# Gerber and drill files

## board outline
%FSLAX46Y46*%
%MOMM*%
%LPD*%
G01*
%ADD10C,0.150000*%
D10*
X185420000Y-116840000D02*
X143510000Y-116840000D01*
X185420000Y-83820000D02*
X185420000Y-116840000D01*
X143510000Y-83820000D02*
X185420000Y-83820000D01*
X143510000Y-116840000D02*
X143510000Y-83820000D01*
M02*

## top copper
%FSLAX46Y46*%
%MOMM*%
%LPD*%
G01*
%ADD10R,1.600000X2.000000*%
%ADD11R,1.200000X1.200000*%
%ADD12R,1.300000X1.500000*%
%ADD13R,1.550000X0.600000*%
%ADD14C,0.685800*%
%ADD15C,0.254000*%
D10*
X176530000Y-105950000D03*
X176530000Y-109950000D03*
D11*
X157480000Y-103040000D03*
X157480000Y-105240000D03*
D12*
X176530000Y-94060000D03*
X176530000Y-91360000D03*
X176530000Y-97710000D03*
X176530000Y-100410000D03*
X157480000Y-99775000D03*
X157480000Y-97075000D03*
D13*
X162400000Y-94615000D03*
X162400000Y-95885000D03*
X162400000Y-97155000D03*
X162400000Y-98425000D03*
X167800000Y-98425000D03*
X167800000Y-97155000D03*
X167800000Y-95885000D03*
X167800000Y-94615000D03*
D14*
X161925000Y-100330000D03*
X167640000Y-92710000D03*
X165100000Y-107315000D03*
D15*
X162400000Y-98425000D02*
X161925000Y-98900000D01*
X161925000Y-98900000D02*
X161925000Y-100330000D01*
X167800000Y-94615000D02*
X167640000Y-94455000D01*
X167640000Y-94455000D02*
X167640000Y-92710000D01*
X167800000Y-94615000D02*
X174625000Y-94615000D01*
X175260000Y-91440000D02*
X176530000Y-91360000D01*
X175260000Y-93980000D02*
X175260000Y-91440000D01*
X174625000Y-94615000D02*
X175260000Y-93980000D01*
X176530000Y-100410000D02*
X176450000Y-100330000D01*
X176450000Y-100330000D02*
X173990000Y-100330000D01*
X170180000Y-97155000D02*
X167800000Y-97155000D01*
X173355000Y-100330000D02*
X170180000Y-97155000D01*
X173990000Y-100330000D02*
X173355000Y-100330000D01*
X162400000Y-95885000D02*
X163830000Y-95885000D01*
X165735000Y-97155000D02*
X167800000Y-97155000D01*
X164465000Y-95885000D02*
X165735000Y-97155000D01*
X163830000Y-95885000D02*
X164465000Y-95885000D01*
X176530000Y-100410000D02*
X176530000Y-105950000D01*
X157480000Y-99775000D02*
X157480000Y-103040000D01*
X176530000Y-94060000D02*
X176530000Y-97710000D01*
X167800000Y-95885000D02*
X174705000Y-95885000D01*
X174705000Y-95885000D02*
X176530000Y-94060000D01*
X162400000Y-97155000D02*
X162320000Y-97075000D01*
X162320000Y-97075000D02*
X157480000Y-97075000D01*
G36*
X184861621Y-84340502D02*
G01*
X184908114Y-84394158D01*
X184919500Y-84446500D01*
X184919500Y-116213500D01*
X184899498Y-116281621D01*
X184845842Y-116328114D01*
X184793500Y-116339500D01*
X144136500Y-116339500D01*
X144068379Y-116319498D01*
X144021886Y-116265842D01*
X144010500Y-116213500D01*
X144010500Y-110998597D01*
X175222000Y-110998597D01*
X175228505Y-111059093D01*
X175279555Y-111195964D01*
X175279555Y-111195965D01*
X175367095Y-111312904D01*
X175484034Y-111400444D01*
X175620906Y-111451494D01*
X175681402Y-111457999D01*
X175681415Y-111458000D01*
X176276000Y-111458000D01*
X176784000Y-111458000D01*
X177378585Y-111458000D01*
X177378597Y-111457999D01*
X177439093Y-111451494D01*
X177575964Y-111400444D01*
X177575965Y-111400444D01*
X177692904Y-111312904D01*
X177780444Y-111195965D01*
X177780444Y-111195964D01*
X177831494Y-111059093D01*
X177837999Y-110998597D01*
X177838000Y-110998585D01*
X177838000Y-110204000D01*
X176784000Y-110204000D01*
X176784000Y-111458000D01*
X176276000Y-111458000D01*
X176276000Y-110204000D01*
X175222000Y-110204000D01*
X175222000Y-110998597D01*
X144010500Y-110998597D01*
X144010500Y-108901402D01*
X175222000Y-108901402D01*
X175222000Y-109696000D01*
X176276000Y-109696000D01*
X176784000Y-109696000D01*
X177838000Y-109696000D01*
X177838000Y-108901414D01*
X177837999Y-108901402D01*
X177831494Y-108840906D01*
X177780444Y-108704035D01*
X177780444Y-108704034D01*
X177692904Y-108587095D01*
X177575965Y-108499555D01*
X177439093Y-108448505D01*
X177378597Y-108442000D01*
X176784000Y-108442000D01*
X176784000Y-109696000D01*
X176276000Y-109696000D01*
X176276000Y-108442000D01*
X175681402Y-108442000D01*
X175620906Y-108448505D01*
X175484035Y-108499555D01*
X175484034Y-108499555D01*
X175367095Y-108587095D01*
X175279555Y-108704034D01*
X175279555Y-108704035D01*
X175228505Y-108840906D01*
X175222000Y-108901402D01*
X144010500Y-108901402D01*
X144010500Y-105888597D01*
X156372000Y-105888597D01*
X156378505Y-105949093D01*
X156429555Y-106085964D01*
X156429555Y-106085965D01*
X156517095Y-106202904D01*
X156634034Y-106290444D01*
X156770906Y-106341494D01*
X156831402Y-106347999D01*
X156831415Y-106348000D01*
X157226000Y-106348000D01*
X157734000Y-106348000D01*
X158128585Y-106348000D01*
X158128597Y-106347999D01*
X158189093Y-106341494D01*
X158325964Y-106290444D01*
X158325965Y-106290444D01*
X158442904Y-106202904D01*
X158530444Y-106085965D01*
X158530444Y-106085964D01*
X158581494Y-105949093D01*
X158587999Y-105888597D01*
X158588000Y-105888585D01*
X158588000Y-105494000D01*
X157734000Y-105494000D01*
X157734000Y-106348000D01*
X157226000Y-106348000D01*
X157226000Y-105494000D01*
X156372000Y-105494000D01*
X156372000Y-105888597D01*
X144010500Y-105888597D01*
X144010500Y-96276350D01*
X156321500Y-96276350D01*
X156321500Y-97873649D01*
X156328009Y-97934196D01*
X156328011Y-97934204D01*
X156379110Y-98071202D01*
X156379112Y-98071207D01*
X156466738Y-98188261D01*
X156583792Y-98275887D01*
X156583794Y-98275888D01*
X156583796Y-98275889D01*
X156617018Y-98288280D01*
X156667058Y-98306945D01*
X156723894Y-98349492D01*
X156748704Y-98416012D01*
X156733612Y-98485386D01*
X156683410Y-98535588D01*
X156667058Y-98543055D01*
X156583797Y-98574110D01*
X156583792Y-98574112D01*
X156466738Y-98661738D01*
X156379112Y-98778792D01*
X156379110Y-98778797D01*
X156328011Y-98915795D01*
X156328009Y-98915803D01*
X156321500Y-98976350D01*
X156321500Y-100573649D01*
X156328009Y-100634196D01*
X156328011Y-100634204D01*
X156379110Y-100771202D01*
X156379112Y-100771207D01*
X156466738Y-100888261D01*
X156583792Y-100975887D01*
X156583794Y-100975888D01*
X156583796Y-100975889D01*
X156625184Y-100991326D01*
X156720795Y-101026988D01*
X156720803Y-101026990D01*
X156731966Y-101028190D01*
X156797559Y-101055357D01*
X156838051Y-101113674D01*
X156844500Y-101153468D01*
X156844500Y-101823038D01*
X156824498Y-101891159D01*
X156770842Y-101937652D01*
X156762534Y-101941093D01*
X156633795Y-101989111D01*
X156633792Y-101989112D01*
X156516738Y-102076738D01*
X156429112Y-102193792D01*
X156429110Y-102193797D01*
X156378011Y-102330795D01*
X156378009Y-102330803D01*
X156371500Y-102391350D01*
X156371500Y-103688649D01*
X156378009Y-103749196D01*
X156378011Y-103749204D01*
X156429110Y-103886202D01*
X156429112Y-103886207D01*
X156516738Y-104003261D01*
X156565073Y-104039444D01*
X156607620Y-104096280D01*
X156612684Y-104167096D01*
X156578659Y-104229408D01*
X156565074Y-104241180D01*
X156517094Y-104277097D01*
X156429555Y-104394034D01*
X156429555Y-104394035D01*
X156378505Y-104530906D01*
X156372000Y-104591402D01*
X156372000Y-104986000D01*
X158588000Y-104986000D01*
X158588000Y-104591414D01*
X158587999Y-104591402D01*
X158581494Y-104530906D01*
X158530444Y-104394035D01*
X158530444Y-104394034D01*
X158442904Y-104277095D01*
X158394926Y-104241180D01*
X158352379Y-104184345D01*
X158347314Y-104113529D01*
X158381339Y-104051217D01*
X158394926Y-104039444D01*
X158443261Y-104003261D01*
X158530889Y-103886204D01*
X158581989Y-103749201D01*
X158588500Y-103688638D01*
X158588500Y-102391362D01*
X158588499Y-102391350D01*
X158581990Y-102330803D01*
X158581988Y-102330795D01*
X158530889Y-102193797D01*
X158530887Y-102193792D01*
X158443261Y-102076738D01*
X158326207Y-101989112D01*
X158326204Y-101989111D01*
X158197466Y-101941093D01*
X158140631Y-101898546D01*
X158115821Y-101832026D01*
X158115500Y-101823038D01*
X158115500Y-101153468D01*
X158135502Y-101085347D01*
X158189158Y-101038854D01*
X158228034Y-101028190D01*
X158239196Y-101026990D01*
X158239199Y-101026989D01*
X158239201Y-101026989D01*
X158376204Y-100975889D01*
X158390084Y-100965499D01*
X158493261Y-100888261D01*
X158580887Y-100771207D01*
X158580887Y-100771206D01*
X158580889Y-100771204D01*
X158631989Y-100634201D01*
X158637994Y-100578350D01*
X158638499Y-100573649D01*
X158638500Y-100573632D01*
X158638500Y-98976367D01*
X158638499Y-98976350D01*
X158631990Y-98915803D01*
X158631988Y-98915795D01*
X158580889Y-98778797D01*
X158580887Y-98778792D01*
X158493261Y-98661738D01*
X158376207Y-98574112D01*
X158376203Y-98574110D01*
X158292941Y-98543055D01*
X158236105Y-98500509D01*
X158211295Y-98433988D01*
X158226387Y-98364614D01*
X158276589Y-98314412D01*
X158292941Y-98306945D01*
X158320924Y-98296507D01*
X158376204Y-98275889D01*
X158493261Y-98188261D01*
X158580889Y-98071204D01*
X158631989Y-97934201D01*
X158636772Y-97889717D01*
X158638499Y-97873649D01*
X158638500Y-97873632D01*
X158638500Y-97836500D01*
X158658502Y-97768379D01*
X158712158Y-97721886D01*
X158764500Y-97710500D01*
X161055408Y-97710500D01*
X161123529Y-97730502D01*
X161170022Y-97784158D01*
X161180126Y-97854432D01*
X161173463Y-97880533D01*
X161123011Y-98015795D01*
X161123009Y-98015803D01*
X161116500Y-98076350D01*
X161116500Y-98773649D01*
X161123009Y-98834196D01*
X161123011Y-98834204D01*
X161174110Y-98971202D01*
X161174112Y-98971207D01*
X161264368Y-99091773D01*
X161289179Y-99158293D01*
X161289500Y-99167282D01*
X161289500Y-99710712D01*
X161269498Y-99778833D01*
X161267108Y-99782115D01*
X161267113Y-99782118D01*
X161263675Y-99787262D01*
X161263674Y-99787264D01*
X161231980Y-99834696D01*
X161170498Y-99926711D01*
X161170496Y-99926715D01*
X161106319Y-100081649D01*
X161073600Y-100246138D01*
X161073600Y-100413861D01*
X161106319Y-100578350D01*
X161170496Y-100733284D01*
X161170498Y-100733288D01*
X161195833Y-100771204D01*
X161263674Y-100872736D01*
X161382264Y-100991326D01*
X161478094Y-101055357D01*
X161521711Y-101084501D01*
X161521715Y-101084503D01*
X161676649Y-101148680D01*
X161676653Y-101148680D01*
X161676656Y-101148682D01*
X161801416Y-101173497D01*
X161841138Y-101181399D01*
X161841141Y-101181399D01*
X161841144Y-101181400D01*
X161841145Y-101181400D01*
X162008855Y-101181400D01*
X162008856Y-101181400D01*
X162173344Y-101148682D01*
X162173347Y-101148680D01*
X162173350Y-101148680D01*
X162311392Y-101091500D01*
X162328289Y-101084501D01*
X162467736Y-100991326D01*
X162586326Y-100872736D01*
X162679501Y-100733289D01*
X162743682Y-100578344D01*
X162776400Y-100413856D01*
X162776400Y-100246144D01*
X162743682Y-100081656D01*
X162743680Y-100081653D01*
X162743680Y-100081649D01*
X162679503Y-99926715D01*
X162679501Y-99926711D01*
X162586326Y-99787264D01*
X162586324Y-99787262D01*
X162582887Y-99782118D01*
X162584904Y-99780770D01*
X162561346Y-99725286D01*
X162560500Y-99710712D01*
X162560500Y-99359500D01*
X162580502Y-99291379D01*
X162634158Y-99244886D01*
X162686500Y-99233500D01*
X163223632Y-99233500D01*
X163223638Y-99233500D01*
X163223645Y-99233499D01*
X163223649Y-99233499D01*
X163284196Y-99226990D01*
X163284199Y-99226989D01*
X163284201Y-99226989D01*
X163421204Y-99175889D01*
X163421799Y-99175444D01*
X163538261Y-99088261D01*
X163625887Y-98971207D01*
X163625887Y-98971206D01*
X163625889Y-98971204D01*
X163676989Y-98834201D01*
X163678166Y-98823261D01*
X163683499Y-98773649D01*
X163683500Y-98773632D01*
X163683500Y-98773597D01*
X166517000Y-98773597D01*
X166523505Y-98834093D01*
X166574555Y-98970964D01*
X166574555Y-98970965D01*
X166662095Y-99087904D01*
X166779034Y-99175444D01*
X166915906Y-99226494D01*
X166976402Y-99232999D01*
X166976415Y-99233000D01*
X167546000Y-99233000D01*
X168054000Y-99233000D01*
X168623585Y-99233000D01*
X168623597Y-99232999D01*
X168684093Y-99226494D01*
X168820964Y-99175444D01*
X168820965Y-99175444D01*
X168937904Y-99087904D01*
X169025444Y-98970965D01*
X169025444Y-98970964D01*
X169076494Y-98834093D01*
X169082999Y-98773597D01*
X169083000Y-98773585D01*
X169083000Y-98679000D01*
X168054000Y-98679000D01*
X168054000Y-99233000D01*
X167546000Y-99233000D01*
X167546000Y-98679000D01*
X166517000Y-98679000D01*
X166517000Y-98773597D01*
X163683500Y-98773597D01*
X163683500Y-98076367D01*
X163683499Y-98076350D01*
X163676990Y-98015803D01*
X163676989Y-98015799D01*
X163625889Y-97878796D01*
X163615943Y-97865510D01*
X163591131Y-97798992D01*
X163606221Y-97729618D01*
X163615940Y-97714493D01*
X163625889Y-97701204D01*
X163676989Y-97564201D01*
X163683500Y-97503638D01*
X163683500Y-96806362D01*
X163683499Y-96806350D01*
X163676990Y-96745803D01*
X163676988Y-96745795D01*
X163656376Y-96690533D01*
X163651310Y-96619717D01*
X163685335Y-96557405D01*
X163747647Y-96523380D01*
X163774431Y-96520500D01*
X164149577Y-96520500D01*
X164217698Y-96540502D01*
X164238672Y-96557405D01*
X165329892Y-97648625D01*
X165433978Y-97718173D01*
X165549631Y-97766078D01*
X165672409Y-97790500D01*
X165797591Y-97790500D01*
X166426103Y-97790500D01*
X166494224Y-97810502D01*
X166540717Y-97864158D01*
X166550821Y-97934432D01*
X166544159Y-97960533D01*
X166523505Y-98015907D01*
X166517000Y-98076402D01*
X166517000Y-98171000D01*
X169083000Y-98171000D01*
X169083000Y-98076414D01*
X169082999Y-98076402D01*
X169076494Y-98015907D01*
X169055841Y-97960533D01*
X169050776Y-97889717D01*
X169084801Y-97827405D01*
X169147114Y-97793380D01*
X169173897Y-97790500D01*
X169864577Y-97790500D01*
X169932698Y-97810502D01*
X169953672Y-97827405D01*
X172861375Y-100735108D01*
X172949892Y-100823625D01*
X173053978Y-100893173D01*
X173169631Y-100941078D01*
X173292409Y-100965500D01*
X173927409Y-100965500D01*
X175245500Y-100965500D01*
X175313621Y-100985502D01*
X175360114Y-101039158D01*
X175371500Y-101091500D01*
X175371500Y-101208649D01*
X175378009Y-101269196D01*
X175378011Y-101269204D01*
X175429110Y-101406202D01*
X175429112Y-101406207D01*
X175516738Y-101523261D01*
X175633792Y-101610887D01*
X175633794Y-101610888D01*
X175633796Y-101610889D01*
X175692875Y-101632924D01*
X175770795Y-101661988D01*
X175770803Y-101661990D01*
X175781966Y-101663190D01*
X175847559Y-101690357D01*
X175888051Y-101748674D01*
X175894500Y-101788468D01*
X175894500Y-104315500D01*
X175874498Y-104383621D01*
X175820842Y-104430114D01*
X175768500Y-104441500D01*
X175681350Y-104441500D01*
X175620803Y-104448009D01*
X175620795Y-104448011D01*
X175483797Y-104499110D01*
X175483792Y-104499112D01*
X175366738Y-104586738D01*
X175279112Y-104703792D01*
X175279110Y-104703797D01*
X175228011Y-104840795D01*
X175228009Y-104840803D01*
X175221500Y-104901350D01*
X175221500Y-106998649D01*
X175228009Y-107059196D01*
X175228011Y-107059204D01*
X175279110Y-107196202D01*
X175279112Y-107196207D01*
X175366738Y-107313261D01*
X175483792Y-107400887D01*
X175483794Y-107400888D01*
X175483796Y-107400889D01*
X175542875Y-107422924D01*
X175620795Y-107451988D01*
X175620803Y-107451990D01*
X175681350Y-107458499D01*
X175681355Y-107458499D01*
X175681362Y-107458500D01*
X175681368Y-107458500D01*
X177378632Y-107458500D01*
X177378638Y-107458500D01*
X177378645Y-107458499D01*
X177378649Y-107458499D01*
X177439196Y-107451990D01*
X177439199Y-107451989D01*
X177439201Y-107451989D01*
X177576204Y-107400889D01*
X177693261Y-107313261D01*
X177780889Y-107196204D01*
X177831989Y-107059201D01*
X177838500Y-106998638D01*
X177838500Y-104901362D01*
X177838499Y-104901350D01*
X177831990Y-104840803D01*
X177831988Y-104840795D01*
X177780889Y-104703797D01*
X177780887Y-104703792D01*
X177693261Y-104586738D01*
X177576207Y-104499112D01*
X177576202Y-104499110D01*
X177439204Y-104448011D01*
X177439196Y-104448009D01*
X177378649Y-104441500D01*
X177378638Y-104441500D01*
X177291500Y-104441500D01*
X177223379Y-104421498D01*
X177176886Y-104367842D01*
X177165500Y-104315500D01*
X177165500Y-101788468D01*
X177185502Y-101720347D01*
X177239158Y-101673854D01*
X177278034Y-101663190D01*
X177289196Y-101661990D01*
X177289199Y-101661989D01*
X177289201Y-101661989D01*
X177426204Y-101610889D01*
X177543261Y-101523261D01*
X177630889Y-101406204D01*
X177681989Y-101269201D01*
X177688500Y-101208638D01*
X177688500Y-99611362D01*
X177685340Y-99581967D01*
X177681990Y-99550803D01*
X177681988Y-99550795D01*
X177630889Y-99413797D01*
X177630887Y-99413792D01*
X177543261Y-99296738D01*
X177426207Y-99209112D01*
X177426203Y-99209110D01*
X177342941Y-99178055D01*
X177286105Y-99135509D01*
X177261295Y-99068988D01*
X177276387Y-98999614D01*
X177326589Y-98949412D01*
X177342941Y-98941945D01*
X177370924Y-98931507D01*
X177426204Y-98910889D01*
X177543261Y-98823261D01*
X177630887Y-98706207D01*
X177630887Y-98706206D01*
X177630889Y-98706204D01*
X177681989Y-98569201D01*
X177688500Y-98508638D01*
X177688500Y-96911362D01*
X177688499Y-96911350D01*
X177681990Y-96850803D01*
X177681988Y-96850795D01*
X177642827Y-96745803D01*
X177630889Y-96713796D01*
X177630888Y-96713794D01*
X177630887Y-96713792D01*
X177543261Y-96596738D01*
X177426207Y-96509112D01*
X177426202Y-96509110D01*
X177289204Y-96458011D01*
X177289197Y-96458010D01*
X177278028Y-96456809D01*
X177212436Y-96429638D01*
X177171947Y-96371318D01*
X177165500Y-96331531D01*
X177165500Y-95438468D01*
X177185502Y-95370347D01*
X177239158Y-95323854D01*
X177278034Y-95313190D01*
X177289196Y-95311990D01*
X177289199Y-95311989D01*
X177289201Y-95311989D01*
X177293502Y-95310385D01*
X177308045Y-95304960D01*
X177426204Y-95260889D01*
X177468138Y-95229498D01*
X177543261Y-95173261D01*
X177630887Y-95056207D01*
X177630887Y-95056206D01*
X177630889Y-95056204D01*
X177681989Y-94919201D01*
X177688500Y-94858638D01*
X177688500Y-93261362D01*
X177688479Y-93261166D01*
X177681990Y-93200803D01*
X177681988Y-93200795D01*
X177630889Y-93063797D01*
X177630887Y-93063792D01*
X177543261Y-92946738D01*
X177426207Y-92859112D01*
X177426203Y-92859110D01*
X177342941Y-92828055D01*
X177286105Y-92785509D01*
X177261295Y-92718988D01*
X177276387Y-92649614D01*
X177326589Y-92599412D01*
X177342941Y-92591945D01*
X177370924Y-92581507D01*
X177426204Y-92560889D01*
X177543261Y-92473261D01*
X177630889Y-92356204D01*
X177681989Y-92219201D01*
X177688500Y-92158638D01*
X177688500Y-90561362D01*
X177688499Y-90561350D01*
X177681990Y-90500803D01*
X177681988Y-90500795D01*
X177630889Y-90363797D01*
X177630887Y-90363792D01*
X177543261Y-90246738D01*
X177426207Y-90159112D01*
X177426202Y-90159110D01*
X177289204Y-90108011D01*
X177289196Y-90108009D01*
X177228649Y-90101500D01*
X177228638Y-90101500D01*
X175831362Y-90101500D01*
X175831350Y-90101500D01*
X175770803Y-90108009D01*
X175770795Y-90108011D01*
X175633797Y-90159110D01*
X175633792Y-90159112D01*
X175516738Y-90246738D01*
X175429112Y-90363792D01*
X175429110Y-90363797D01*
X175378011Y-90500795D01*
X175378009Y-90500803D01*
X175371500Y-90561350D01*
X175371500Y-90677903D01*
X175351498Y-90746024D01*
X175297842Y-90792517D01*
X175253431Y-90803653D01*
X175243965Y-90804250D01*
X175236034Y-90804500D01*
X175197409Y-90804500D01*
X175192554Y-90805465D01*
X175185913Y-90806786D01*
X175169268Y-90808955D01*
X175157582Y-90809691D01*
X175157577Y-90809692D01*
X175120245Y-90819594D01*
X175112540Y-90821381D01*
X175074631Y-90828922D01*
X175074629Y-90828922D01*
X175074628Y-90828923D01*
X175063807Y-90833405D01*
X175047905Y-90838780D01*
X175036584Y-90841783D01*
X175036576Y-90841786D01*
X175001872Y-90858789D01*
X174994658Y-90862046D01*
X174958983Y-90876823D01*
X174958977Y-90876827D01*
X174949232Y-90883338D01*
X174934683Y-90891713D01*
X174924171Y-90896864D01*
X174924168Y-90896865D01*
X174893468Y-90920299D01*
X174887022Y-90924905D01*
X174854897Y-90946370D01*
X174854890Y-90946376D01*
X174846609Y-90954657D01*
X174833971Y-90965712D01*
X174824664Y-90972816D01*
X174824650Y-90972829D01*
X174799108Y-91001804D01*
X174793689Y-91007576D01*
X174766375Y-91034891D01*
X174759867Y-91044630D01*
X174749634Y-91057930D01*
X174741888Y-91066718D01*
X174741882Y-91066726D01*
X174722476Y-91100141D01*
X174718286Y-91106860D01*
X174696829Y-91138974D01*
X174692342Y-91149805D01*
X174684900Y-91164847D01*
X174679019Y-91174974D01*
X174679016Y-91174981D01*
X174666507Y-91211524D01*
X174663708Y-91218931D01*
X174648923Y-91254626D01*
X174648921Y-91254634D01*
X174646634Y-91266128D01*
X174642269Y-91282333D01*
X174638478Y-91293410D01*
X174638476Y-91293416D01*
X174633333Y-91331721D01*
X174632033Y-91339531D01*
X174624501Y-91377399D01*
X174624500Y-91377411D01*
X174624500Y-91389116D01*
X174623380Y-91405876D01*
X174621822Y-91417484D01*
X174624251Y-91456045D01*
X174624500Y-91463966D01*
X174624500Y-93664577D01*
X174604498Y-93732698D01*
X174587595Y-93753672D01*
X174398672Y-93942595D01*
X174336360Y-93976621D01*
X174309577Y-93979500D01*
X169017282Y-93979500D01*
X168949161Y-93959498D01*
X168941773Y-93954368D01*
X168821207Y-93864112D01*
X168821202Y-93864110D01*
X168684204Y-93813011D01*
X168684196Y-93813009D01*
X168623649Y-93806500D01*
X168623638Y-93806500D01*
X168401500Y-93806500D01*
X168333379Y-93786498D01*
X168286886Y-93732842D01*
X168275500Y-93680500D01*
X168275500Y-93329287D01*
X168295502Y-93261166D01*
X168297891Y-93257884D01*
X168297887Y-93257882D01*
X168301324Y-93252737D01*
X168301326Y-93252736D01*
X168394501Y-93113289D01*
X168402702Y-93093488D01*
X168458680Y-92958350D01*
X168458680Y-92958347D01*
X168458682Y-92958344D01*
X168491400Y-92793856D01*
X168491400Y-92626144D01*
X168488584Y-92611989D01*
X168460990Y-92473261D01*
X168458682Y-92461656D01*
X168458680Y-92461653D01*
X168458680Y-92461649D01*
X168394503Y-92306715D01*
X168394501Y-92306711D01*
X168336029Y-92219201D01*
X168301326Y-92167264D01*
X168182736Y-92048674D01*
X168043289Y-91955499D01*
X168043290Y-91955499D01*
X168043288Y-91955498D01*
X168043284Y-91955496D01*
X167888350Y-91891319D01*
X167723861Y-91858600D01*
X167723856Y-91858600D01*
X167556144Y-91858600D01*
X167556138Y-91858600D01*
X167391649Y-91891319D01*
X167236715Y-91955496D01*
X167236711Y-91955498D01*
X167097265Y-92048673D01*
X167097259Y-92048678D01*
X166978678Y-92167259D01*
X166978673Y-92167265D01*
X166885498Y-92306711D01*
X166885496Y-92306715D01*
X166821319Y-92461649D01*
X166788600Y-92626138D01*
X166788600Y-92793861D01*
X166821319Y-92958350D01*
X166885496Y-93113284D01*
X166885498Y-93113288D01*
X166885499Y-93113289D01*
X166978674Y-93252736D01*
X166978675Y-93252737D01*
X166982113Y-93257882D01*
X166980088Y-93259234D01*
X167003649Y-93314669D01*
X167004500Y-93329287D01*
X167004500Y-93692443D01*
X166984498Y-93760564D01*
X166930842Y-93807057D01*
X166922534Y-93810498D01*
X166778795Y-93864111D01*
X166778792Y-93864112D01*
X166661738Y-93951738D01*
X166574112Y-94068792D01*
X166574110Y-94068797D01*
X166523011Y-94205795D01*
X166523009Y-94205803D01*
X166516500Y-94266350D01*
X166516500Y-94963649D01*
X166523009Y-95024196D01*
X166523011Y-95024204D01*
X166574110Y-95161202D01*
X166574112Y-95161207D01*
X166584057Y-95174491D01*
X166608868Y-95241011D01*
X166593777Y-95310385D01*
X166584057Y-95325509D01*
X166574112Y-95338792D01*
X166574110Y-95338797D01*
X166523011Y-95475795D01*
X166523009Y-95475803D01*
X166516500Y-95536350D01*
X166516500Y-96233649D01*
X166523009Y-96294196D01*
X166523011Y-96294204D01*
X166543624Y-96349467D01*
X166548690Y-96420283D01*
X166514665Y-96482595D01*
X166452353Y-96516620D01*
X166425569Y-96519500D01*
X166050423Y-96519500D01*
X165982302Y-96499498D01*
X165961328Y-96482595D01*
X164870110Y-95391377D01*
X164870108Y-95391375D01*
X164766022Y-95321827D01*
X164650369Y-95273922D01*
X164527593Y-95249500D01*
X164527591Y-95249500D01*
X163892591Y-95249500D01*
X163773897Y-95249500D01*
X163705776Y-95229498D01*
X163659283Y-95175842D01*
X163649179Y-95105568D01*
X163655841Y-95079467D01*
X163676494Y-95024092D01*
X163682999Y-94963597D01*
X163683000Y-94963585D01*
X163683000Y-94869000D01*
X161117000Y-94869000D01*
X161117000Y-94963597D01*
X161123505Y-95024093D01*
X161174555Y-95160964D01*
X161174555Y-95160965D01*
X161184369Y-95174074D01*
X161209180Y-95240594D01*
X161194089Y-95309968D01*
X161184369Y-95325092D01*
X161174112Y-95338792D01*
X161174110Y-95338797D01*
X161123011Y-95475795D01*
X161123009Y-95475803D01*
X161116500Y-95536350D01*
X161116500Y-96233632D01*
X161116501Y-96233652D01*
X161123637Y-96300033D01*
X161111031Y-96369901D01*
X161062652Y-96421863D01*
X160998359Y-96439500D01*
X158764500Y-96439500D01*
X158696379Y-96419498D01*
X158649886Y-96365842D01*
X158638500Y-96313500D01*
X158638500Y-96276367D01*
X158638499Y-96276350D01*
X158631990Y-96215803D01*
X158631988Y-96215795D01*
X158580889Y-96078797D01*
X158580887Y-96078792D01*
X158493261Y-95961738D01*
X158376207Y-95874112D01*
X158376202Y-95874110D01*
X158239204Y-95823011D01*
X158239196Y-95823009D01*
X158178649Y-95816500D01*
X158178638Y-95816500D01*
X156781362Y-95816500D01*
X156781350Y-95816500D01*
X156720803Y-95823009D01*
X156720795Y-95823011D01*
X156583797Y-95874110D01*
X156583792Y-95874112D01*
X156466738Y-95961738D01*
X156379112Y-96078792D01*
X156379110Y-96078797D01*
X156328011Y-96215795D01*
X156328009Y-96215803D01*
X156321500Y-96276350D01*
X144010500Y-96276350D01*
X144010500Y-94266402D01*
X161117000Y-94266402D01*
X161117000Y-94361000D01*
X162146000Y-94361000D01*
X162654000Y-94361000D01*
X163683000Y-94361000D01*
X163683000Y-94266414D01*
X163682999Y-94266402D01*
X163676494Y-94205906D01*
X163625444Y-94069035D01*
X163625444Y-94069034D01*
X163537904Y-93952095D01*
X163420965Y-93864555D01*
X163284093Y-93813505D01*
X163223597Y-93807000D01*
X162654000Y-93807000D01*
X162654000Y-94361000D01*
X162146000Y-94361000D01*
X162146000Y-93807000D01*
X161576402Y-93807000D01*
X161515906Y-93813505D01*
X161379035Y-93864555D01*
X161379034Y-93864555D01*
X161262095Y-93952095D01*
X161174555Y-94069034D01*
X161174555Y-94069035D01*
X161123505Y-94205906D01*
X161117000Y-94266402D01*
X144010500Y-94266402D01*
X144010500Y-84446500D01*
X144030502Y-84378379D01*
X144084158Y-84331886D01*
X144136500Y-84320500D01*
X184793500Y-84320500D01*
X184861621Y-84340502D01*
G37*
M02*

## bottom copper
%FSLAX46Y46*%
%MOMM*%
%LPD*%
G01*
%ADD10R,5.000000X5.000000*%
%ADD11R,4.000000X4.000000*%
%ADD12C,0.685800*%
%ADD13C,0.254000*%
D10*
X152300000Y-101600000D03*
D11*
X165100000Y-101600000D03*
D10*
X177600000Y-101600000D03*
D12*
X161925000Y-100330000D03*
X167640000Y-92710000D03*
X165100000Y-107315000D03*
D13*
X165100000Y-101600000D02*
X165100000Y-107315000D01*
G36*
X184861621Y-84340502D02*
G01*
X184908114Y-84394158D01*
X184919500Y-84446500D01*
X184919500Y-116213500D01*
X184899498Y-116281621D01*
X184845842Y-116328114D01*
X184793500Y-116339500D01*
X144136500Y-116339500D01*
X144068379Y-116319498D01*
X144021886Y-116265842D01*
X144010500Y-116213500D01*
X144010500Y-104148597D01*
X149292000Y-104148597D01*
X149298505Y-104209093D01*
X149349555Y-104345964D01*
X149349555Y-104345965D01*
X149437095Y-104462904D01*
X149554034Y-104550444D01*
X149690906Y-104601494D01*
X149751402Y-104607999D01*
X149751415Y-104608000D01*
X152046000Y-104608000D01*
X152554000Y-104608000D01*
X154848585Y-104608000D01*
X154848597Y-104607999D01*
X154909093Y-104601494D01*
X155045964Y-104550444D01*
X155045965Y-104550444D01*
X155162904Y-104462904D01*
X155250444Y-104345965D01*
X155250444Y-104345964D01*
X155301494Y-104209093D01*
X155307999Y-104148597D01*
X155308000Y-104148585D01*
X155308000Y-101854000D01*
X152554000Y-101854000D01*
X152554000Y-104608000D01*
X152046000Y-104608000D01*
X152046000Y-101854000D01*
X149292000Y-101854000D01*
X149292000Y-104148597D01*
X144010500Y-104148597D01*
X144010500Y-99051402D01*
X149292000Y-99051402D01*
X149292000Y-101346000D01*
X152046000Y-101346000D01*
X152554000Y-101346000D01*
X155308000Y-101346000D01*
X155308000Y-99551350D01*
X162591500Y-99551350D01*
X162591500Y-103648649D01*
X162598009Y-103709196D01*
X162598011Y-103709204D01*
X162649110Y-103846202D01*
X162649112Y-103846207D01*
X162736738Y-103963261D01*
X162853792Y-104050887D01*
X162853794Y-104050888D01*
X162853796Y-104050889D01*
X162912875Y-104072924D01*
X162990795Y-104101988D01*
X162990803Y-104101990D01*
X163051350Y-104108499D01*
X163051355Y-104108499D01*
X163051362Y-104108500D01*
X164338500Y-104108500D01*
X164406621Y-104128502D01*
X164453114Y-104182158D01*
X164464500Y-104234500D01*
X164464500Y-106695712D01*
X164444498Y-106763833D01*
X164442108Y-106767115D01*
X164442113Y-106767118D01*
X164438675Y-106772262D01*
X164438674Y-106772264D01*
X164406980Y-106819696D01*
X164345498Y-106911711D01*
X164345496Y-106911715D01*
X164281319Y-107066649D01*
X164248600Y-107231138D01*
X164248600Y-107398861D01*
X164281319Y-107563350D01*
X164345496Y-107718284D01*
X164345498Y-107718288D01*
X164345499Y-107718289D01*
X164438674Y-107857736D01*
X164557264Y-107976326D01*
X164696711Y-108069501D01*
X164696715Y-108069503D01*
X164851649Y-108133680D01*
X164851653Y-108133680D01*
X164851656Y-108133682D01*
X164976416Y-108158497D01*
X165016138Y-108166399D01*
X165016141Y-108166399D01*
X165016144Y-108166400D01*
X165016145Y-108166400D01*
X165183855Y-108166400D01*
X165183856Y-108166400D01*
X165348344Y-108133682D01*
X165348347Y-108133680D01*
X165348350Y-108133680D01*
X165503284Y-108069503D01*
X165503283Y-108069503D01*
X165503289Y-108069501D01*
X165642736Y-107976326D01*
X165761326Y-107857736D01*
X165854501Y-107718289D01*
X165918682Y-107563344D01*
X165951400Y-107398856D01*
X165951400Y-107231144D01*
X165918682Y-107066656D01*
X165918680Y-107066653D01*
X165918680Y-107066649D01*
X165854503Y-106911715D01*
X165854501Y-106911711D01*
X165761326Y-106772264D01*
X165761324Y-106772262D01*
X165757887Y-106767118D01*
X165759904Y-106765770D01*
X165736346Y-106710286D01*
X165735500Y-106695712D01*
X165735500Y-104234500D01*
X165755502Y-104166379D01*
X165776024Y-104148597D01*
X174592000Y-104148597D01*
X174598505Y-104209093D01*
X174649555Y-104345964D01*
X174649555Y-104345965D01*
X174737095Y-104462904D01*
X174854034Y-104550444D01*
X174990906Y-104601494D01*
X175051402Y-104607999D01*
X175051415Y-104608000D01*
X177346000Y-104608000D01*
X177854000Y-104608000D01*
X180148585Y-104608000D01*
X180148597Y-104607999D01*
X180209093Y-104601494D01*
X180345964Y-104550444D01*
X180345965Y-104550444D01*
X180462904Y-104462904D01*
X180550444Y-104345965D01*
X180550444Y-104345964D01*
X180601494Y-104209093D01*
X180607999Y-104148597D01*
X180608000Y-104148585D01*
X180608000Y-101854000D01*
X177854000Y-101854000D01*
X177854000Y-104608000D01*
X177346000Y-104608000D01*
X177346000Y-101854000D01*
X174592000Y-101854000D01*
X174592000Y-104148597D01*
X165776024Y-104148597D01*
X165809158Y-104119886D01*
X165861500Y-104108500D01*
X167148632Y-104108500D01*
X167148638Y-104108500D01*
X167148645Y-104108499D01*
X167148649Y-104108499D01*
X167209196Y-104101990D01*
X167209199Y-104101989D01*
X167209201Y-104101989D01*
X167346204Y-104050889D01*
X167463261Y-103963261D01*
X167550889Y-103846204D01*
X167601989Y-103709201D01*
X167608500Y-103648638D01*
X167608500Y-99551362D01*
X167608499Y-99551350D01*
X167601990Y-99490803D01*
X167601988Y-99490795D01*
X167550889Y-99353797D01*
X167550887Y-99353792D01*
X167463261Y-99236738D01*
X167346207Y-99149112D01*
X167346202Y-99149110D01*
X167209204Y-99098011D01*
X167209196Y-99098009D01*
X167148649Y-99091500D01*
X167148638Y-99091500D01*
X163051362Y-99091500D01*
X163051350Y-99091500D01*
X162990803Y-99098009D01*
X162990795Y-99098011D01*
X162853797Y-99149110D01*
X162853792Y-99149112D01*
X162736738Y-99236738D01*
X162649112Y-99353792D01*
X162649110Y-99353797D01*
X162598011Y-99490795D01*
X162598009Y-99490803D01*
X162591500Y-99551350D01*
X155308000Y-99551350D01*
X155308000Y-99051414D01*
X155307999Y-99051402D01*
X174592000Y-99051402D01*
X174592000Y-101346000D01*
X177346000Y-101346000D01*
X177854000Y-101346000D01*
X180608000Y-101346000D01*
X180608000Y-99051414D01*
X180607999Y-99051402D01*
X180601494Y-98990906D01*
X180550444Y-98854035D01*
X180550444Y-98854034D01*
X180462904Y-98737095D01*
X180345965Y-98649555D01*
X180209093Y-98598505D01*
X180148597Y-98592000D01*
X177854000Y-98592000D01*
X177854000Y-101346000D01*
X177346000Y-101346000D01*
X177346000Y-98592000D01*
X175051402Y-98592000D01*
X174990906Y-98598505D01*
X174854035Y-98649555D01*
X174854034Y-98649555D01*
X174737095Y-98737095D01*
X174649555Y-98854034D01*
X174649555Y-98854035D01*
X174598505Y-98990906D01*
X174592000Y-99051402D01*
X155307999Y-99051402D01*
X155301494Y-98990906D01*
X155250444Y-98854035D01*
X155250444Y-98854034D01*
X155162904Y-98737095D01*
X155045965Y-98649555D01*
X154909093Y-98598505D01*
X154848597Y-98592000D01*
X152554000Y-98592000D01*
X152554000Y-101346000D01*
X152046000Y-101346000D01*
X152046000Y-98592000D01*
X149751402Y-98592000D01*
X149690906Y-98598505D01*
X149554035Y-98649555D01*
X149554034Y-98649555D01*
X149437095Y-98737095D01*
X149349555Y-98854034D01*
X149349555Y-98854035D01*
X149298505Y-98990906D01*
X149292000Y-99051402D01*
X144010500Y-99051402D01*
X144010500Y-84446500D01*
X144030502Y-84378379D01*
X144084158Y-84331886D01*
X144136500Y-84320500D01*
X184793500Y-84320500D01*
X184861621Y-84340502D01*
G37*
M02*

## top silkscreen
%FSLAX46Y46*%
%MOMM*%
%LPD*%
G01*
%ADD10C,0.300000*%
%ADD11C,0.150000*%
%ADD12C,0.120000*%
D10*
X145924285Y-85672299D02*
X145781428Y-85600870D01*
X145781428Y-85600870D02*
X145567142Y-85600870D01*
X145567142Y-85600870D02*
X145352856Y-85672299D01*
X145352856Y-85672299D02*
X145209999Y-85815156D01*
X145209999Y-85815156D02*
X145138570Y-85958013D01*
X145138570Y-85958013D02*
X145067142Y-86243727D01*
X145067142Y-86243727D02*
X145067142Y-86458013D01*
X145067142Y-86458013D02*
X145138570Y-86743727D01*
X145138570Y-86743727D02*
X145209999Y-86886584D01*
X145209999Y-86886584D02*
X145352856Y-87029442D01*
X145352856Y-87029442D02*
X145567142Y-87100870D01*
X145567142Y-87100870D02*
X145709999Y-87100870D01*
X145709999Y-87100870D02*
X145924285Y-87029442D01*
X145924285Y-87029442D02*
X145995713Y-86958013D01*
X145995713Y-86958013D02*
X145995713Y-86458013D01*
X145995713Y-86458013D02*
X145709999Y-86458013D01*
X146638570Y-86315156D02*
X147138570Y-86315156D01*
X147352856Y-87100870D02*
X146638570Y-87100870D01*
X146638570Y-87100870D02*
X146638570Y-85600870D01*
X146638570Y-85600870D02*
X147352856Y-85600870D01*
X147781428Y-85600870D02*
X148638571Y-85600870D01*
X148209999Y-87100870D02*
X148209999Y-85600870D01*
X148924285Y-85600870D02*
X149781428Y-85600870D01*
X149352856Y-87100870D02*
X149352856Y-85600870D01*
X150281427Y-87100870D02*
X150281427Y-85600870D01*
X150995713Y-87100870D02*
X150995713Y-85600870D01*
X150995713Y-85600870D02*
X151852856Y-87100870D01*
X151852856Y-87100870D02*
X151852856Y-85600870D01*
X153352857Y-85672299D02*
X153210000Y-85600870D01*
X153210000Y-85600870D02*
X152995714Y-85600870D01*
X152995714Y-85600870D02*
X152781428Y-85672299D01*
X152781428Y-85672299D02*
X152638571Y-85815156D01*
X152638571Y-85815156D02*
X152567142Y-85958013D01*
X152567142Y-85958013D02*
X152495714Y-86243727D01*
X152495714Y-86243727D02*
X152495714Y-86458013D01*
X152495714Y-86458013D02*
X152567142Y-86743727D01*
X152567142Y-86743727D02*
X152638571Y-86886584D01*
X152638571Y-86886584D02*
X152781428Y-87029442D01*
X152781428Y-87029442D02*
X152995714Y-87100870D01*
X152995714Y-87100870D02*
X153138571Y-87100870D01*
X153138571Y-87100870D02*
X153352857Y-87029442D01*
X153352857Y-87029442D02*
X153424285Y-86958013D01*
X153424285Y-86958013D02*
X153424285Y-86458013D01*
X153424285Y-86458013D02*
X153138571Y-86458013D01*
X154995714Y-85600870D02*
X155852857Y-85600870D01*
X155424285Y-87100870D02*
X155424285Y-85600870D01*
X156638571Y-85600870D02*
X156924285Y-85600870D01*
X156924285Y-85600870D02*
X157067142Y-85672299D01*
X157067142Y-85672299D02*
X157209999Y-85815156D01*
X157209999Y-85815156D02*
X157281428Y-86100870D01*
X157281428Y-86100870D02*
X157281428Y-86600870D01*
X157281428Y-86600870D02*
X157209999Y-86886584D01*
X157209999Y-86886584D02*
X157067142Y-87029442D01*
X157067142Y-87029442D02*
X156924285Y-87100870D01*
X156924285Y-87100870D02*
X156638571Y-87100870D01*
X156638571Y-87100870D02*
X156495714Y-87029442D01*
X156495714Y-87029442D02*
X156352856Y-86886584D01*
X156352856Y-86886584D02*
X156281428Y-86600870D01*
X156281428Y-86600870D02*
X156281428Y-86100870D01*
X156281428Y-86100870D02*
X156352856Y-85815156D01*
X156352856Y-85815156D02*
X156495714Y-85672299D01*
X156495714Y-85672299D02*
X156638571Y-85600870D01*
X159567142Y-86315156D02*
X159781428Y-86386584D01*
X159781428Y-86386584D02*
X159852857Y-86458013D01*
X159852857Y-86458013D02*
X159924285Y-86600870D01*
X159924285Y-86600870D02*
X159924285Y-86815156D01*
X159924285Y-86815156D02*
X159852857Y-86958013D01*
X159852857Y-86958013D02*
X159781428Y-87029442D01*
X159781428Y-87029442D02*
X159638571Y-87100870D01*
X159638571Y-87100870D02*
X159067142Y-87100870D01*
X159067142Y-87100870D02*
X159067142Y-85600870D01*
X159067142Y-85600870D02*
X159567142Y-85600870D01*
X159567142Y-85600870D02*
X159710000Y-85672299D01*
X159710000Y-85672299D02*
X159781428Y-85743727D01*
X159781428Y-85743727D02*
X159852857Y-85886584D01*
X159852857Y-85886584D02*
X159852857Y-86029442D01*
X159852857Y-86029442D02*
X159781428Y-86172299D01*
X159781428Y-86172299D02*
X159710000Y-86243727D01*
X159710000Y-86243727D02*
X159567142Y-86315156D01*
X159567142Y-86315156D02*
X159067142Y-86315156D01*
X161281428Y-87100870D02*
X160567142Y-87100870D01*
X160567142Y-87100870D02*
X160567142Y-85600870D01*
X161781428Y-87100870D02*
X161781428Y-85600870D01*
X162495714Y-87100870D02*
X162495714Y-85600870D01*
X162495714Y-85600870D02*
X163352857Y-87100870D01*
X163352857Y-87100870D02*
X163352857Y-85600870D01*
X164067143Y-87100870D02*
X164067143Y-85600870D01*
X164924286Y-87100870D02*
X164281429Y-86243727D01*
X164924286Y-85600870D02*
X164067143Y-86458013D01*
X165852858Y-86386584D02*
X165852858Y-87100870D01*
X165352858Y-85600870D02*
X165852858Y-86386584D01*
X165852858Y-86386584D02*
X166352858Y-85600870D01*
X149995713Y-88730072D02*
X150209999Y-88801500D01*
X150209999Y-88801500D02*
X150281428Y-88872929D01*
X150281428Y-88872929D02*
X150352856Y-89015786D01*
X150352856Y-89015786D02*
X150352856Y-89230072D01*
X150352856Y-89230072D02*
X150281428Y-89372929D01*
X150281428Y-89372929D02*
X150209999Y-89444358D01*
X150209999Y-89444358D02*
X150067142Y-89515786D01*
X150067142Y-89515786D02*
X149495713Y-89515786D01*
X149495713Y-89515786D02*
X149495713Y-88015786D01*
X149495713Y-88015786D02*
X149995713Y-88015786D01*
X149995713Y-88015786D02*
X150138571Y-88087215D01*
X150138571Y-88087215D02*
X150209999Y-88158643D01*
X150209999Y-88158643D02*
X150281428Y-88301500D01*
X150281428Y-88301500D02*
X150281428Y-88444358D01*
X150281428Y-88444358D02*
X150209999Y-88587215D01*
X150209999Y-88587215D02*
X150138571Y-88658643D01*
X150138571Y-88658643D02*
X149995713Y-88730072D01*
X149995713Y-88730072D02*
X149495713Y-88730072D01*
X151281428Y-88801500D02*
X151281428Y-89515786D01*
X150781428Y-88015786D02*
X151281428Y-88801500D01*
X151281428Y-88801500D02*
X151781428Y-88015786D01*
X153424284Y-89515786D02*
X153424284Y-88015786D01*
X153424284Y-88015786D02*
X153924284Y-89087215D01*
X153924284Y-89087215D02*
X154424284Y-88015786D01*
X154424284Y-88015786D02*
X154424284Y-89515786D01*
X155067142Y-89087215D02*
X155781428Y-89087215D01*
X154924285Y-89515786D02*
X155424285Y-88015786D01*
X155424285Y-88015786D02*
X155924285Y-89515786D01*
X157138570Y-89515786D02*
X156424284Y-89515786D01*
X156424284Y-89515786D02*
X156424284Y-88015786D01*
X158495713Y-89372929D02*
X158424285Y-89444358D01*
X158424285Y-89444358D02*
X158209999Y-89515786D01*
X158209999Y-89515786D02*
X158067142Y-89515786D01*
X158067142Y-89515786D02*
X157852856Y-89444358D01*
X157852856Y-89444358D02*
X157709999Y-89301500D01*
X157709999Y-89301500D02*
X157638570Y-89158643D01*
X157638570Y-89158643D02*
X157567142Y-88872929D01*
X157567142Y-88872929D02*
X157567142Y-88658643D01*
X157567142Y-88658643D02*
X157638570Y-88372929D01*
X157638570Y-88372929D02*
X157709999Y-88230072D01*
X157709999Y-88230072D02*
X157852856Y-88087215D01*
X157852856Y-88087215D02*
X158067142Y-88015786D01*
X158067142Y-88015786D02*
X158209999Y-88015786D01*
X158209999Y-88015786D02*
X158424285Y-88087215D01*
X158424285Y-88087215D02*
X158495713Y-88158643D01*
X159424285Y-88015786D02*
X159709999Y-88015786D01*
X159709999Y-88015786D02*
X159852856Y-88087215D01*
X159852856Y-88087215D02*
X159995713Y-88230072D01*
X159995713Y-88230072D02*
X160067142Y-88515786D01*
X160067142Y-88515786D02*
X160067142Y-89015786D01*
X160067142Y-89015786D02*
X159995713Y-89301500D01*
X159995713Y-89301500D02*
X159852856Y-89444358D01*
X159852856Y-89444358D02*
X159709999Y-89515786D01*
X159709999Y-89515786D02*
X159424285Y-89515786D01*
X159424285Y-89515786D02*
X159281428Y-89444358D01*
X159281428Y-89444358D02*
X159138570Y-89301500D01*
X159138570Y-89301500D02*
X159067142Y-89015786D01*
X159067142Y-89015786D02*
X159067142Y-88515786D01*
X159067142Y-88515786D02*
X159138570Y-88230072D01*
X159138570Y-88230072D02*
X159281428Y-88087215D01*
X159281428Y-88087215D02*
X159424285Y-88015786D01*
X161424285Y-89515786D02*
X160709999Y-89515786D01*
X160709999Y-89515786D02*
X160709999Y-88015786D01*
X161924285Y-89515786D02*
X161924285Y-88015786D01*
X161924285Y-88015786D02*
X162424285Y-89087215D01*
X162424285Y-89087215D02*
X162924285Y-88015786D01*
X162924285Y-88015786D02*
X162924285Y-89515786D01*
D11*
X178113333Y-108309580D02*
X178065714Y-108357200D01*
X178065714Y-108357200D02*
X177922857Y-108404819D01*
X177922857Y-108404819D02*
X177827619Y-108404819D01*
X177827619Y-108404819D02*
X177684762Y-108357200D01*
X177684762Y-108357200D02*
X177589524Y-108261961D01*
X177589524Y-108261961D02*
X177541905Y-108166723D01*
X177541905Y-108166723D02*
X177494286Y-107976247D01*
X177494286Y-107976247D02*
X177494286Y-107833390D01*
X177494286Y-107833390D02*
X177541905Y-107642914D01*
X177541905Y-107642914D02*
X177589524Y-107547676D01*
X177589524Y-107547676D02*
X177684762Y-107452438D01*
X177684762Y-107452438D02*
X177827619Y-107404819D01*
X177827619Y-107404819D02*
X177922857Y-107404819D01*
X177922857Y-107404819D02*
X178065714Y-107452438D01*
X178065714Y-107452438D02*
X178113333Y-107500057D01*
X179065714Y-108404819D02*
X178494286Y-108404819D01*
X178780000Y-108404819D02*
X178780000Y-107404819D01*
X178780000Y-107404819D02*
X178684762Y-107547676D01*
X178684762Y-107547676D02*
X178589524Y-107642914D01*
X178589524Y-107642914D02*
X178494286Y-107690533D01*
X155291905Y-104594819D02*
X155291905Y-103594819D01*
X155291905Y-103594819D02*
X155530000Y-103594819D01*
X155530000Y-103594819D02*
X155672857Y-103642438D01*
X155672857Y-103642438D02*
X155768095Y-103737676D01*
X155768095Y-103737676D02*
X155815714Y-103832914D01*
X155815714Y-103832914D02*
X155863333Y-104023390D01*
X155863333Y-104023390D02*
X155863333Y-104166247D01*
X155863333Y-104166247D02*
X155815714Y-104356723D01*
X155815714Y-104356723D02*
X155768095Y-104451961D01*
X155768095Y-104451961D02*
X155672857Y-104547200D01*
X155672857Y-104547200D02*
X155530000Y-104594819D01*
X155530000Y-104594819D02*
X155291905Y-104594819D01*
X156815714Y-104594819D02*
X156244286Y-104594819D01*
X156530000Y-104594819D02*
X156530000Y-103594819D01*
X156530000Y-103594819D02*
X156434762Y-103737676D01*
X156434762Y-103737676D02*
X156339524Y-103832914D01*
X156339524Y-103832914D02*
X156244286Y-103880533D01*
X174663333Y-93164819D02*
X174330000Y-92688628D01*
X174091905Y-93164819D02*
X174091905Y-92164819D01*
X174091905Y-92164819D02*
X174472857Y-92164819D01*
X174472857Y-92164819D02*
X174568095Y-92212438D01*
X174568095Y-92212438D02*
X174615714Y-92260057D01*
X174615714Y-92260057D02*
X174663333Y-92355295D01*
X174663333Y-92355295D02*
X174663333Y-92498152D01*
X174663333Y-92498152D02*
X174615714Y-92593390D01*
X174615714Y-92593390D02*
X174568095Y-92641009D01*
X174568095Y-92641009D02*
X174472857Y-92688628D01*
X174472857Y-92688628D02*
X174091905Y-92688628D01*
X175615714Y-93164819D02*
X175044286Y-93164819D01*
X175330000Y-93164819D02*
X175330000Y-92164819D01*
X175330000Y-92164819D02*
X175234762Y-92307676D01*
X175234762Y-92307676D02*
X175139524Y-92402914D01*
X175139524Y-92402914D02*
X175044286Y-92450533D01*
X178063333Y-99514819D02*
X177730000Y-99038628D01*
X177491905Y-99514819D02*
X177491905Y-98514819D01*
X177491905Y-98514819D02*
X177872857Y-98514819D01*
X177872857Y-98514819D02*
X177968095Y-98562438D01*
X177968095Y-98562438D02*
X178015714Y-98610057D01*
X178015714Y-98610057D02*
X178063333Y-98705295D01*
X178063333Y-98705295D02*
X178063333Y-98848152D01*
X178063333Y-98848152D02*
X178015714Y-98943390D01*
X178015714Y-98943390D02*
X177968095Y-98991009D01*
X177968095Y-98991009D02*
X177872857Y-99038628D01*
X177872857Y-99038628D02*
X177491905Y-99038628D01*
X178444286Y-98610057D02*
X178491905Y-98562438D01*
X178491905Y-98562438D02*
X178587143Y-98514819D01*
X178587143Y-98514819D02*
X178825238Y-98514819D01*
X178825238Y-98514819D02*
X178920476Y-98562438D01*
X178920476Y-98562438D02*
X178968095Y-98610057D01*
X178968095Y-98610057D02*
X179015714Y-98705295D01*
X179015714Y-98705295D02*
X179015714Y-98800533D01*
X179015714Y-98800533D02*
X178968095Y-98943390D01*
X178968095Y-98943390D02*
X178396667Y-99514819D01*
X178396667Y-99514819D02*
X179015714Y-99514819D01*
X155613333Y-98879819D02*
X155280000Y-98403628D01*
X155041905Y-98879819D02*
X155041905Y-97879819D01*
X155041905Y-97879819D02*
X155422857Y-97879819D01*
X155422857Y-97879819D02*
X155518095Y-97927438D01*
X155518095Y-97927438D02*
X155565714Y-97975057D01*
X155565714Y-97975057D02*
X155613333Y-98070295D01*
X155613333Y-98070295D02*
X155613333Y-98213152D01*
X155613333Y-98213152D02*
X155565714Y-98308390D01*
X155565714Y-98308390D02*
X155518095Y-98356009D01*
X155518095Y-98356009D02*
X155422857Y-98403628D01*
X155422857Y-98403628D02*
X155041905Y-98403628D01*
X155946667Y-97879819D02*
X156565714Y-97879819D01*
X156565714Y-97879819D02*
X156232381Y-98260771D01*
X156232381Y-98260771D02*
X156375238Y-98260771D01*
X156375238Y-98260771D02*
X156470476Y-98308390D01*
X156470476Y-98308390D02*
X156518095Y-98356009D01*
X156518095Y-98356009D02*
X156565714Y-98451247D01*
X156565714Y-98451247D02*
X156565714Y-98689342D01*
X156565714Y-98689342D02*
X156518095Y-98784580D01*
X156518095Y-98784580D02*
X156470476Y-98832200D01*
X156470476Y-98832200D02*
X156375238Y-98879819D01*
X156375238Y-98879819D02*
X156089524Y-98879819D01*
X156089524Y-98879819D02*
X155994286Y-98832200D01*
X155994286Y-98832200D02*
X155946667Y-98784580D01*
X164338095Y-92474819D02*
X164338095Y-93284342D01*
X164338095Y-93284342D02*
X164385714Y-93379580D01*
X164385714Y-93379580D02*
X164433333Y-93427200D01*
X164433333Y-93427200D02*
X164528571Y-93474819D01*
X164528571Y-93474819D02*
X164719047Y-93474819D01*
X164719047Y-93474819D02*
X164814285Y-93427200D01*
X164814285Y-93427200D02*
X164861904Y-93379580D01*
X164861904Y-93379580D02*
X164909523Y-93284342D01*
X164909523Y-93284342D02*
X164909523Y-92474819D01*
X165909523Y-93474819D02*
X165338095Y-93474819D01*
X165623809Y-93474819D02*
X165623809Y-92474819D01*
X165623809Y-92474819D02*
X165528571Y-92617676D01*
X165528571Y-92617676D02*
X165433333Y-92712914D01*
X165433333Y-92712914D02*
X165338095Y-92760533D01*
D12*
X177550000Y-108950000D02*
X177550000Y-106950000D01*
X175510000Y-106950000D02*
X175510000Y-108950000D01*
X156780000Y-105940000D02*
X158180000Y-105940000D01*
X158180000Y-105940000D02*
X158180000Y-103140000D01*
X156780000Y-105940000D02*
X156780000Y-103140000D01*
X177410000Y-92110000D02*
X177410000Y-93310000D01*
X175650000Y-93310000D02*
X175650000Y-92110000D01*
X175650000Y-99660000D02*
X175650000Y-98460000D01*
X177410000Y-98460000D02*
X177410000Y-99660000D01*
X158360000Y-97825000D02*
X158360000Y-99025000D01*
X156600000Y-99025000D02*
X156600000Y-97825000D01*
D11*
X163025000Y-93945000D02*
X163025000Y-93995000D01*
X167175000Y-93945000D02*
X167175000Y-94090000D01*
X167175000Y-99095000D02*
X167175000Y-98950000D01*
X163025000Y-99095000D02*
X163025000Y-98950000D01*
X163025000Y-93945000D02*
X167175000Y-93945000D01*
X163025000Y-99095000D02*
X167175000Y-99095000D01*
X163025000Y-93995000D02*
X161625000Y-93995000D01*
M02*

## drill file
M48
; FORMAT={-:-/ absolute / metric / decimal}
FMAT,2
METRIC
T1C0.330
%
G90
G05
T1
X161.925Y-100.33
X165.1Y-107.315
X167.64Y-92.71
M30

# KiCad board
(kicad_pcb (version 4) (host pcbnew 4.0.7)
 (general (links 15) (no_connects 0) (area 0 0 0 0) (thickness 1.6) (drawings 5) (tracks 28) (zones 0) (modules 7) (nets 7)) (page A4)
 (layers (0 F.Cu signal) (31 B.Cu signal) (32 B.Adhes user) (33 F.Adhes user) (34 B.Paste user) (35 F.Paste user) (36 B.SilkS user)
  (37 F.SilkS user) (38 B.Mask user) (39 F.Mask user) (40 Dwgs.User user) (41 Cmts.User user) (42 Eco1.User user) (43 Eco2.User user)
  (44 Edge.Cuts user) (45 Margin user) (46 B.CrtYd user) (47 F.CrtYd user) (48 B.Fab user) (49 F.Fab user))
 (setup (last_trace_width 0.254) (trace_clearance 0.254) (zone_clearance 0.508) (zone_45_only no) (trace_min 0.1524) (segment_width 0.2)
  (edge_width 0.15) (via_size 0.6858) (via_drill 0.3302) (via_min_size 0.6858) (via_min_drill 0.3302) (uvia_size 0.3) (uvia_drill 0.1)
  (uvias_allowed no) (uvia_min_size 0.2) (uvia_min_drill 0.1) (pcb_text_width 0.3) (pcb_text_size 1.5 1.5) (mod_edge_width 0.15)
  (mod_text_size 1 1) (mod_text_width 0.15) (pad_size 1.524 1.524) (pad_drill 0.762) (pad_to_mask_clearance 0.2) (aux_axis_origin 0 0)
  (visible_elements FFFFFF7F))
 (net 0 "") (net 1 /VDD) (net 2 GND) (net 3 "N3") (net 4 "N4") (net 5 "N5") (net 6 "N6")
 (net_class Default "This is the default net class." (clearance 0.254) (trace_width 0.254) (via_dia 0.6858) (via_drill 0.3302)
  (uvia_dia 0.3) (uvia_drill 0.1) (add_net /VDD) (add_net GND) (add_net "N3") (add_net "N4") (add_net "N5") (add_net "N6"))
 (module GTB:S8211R (layer B.Cu) (at 165.1 101.6)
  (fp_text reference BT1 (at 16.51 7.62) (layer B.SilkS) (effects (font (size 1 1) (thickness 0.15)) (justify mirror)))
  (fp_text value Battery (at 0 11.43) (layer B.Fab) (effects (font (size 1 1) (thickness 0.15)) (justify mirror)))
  (pad 1 smd rect (at -12.8 0) (size 5 5) (layers B.Cu B.Paste B.Mask) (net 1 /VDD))
  (pad 2 smd rect (at 0 0) (size 4 4) (layers B.Cu B.Paste B.Mask) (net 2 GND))
  (pad 1 smd rect (at 12.5 0) (size 5 5) (layers B.Cu B.Paste B.Mask) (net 1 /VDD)))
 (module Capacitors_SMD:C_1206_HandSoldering (layer F.Cu) (at 176.53 107.95 270)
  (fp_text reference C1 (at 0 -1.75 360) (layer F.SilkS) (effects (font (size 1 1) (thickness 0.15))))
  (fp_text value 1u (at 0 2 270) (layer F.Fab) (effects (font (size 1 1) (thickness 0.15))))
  (fp_line (start 1 -1.02) (end -1 -1.02) (layer F.SilkS) (width 0.12))
  (fp_line (start -1 1.02) (end 1 1.02) (layer F.SilkS) (width 0.12))
  (pad 1 smd rect (at -2 0 270) (size 2 1.6) (layers F.Cu F.Paste F.Mask) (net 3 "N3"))
  (pad 2 smd rect (at 2 0 270) (size 2 1.6) (layers F.Cu F.Paste F.Mask) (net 2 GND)))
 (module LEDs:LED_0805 (layer F.Cu) (at 157.48 104.14 90)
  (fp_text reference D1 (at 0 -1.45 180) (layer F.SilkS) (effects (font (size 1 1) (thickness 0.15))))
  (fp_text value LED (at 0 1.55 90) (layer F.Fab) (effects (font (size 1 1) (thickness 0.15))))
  (fp_line (start -1.8 -0.7) (end -1.8 0.7) (layer F.SilkS) (width 0.12))
  (fp_line (start -1.8 0.7) (end 1 0.7) (layer F.SilkS) (width 0.12))
  (fp_line (start -1.8 -0.7) (end 1 -0.7) (layer F.SilkS) (width 0.12))
  (pad 2 smd rect (at 1.1 0 270) (size 1.2 1.2) (layers F.Cu F.Paste F.Mask) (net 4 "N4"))
  (pad 1 smd rect (at -1.1 0 270) (size 1.2 1.2) (layers F.Cu F.Paste F.Mask) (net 2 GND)))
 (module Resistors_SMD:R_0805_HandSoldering (layer F.Cu) (at 176.53 92.71 90)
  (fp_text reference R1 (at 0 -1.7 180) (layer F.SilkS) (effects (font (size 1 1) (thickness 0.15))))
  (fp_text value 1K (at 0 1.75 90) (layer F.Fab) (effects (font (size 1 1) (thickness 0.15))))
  (fp_line (start 0.6 0.88) (end -0.6 0.88) (layer F.SilkS) (width 0.12))
  (fp_line (start -0.6 -0.88) (end 0.6 -0.88) (layer F.SilkS) (width 0.12))
  (pad 1 smd rect (at -1.35 0 90) (size 1.5 1.3) (layers F.Cu F.Paste F.Mask) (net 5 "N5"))
  (pad 2 smd rect (at 1.35 0 90) (size 1.5 1.3) (layers F.Cu F.Paste F.Mask) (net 1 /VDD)))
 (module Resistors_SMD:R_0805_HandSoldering (layer F.Cu) (at 176.53 99.06 270)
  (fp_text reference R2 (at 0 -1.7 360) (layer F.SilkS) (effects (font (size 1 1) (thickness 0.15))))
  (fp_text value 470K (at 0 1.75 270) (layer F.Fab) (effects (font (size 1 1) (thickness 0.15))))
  (fp_line (start 0.6 0.88) (end -0.6 0.88) (layer F.SilkS) (width 0.12))
  (fp_line (start -0.6 -0.88) (end 0.6 -0.88) (layer F.SilkS) (width 0.12))
  (pad 1 smd rect (at -1.35 0 270) (size 1.5 1.3) (layers F.Cu F.Paste F.Mask) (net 5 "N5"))
  (pad 2 smd rect (at 1.35 0 270) (size 1.5 1.3) (layers F.Cu F.Paste F.Mask) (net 3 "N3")))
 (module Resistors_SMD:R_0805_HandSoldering (layer F.Cu) (at 157.48 98.425 90)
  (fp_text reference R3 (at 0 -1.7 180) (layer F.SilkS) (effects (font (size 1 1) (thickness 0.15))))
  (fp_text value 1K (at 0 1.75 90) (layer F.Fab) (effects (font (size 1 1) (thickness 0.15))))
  (fp_line (start 0.6 0.88) (end -0.6 0.88) (layer F.SilkS) (width 0.12))
  (fp_line (start -0.6 -0.88) (end 0.6 -0.88) (layer F.SilkS) (width 0.12))
  (pad 1 smd rect (at -1.35 0 90) (size 1.5 1.3) (layers F.Cu F.Paste F.Mask) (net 4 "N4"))
  (pad 2 smd rect (at 1.35 0 90) (size 1.5 1.3) (layers F.Cu F.Paste F.Mask) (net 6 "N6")))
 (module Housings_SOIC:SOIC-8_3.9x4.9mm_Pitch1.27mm (layer F.Cu) (at 165.1 96.52)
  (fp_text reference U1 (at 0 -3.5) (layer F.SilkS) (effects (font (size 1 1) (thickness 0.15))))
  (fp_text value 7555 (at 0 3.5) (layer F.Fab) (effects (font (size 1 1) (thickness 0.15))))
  (fp_line (start -2.075 -2.575) (end -2.075 -2.525) (layer F.SilkS) (width 0.15))
  (fp_line (start 2.075 -2.575) (end 2.075 -2.43) (layer F.SilkS) (width 0.15))
  (fp_line (start 2.075 2.575) (end 2.075 2.43) (layer F.SilkS) (width 0.15))
  (fp_line (start -2.075 2.575) (end -2.075 2.43) (layer F.SilkS) (width 0.15))
  (fp_line (start -2.075 -2.575) (end 2.075 -2.575) (layer F.SilkS) (width 0.15))
  (fp_line (start -2.075 2.575) (end 2.075 2.575) (layer F.SilkS) (width 0.15))
  (fp_line (start -2.075 -2.525) (end -3.475 -2.525) (layer F.SilkS) (width 0.15))
  (pad 1 smd rect (at -2.7 -1.905) (size 1.55 0.6) (layers F.Cu F.Paste F.Mask) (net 2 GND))
  (pad 2 smd rect (at -2.7 -0.635) (size 1.55 0.6) (layers F.Cu F.Paste F.Mask) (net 3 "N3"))
  (pad 3 smd rect (at -2.7 0.635) (size 1.55 0.6) (layers F.Cu F.Paste F.Mask) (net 6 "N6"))
  (pad 4 smd rect (at -2.7 1.905) (size 1.55 0.6) (layers F.Cu F.Paste F.Mask) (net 1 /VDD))
  (pad 5 smd rect (at 2.7 1.905) (size 1.55 0.6) (layers F.Cu F.Paste F.Mask) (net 2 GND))
  (pad 6 smd rect (at 2.7 0.635) (size 1.55 0.6) (layers F.Cu F.Paste F.Mask) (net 3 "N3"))
  (pad 7 smd rect (at 2.7 -0.635) (size 1.55 0.6) (layers F.Cu F.Paste F.Mask) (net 5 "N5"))
  (pad 8 smd rect (at 2.7 -1.905) (size 1.55 0.6) (layers F.Cu F.Paste F.Mask) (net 1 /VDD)))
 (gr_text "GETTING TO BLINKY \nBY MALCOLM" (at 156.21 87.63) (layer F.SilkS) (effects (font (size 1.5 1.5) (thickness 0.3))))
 (gr_line (start 185.42 116.84) (end 143.51 116.84) (angle 90) (layer Edge.Cuts) (width 0.15))
 (gr_line (start 185.42 83.82) (end 185.42 116.84) (angle 90) (layer Edge.Cuts) (width 0.15))
 (gr_line (start 143.51 83.82) (end 185.42 83.82) (angle 90) (layer Edge.Cuts) (width 0.15))
 (gr_line (start 143.51 116.84) (end 143.51 83.82) (angle 90) (layer Edge.Cuts) (width 0.15))
 (segment (start 162.4 98.425) (end 161.925 98.9) (width 0.254) (layer F.Cu) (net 1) (status 400000))
 (via (at 161.925 100.33) (size 0.6858) (drill 0.3302) (layers F.Cu B.Cu) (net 1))
 (segment (start 161.925 98.9) (end 161.925 100.33) (width 0.254) (layer F.Cu) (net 1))
 (segment (start 167.8 94.615) (end 167.64 94.455) (width 0.254) (layer F.Cu) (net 1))
 (segment (start 167.64 94.455) (end 167.64 92.71) (width 0.254) (layer F.Cu) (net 1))
 (via (at 167.64 92.71) (size 0.6858) (drill 0.3302) (layers F.Cu B.Cu) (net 1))
 (segment (start 167.8 94.615) (end 174.625 94.615) (width 0.254) (layer F.Cu) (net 1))
 (segment (start 175.26 91.44) (end 176.53 91.36) (width 0.254) (layer F.Cu) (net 1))
 (segment (start 175.26 93.98) (end 175.26 91.44) (width 0.254) (layer F.Cu) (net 1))
 (segment (start 174.625 94.615) (end 175.26 93.98) (width 0.254) (layer F.Cu) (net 1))
 (segment (start 165.1 101.6) (end 165.1 107.315) (width 0.254) (layer B.Cu) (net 2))
 (via (at 165.1 107.315) (size 0.6858) (drill 0.3302) (layers F.Cu B.Cu) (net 2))
 (segment (start 176.53 100.41) (end 176.45 100.33) (width 0.254) (layer F.Cu) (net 3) (status C00000))
 (segment (start 176.45 100.33) (end 173.99 100.33) (width 0.254) (layer F.Cu) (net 3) (status 400000))
 (segment (start 170.18 97.155) (end 167.8 97.155) (width 0.254) (layer F.Cu) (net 3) (status 800000))
 (segment (start 173.355 100.33) (end 170.18 97.155) (width 0.254) (layer F.Cu) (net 3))
 (segment (start 173.99 100.33) (end 173.355 100.33) (width 0.254) (layer F.Cu) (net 3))
 (segment (start 162.4 95.885) (end 163.83 95.885) (width 0.254) (layer F.Cu) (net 3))
 (segment (start 165.735 97.155) (end 167.8 97.155) (width 0.254) (layer F.Cu) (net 3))
 (segment (start 164.465 95.885) (end 165.735 97.155) (width 0.254) (layer F.Cu) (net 3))
 (segment (start 163.83 95.885) (end 164.465 95.885) (width 0.254) (layer F.Cu) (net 3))
 (segment (start 176.53 100.41) (end 176.53 105.95) (width 0.254) (layer F.Cu) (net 3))
 (segment (start 157.48 99.775) (end 157.48 103.04) (width 0.254) (layer F.Cu) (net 4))
 (segment (start 176.53 94.06) (end 176.53 97.71) (width 0.254) (layer F.Cu) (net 5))
 (segment (start 167.8 95.885) (end 174.705 95.885) (width 0.254) (layer F.Cu) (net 5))
 (segment (start 174.705 95.885) (end 176.53 94.06) (width 0.254) (layer F.Cu) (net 5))
 (segment (start 162.4 97.155) (end 162.32 97.075) (width 0.254) (layer F.Cu) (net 6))
 (segment (start 162.32 97.075) (end 157.48 97.075) (width 0.254) (layer F.Cu) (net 6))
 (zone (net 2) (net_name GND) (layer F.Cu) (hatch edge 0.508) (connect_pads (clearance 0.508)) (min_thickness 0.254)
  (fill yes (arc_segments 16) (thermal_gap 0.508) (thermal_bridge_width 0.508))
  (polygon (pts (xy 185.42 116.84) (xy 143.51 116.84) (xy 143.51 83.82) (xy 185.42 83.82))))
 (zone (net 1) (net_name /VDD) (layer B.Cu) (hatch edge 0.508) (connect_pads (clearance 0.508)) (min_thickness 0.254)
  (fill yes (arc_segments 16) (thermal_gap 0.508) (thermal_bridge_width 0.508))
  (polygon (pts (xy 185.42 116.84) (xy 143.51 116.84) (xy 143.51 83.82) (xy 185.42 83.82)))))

